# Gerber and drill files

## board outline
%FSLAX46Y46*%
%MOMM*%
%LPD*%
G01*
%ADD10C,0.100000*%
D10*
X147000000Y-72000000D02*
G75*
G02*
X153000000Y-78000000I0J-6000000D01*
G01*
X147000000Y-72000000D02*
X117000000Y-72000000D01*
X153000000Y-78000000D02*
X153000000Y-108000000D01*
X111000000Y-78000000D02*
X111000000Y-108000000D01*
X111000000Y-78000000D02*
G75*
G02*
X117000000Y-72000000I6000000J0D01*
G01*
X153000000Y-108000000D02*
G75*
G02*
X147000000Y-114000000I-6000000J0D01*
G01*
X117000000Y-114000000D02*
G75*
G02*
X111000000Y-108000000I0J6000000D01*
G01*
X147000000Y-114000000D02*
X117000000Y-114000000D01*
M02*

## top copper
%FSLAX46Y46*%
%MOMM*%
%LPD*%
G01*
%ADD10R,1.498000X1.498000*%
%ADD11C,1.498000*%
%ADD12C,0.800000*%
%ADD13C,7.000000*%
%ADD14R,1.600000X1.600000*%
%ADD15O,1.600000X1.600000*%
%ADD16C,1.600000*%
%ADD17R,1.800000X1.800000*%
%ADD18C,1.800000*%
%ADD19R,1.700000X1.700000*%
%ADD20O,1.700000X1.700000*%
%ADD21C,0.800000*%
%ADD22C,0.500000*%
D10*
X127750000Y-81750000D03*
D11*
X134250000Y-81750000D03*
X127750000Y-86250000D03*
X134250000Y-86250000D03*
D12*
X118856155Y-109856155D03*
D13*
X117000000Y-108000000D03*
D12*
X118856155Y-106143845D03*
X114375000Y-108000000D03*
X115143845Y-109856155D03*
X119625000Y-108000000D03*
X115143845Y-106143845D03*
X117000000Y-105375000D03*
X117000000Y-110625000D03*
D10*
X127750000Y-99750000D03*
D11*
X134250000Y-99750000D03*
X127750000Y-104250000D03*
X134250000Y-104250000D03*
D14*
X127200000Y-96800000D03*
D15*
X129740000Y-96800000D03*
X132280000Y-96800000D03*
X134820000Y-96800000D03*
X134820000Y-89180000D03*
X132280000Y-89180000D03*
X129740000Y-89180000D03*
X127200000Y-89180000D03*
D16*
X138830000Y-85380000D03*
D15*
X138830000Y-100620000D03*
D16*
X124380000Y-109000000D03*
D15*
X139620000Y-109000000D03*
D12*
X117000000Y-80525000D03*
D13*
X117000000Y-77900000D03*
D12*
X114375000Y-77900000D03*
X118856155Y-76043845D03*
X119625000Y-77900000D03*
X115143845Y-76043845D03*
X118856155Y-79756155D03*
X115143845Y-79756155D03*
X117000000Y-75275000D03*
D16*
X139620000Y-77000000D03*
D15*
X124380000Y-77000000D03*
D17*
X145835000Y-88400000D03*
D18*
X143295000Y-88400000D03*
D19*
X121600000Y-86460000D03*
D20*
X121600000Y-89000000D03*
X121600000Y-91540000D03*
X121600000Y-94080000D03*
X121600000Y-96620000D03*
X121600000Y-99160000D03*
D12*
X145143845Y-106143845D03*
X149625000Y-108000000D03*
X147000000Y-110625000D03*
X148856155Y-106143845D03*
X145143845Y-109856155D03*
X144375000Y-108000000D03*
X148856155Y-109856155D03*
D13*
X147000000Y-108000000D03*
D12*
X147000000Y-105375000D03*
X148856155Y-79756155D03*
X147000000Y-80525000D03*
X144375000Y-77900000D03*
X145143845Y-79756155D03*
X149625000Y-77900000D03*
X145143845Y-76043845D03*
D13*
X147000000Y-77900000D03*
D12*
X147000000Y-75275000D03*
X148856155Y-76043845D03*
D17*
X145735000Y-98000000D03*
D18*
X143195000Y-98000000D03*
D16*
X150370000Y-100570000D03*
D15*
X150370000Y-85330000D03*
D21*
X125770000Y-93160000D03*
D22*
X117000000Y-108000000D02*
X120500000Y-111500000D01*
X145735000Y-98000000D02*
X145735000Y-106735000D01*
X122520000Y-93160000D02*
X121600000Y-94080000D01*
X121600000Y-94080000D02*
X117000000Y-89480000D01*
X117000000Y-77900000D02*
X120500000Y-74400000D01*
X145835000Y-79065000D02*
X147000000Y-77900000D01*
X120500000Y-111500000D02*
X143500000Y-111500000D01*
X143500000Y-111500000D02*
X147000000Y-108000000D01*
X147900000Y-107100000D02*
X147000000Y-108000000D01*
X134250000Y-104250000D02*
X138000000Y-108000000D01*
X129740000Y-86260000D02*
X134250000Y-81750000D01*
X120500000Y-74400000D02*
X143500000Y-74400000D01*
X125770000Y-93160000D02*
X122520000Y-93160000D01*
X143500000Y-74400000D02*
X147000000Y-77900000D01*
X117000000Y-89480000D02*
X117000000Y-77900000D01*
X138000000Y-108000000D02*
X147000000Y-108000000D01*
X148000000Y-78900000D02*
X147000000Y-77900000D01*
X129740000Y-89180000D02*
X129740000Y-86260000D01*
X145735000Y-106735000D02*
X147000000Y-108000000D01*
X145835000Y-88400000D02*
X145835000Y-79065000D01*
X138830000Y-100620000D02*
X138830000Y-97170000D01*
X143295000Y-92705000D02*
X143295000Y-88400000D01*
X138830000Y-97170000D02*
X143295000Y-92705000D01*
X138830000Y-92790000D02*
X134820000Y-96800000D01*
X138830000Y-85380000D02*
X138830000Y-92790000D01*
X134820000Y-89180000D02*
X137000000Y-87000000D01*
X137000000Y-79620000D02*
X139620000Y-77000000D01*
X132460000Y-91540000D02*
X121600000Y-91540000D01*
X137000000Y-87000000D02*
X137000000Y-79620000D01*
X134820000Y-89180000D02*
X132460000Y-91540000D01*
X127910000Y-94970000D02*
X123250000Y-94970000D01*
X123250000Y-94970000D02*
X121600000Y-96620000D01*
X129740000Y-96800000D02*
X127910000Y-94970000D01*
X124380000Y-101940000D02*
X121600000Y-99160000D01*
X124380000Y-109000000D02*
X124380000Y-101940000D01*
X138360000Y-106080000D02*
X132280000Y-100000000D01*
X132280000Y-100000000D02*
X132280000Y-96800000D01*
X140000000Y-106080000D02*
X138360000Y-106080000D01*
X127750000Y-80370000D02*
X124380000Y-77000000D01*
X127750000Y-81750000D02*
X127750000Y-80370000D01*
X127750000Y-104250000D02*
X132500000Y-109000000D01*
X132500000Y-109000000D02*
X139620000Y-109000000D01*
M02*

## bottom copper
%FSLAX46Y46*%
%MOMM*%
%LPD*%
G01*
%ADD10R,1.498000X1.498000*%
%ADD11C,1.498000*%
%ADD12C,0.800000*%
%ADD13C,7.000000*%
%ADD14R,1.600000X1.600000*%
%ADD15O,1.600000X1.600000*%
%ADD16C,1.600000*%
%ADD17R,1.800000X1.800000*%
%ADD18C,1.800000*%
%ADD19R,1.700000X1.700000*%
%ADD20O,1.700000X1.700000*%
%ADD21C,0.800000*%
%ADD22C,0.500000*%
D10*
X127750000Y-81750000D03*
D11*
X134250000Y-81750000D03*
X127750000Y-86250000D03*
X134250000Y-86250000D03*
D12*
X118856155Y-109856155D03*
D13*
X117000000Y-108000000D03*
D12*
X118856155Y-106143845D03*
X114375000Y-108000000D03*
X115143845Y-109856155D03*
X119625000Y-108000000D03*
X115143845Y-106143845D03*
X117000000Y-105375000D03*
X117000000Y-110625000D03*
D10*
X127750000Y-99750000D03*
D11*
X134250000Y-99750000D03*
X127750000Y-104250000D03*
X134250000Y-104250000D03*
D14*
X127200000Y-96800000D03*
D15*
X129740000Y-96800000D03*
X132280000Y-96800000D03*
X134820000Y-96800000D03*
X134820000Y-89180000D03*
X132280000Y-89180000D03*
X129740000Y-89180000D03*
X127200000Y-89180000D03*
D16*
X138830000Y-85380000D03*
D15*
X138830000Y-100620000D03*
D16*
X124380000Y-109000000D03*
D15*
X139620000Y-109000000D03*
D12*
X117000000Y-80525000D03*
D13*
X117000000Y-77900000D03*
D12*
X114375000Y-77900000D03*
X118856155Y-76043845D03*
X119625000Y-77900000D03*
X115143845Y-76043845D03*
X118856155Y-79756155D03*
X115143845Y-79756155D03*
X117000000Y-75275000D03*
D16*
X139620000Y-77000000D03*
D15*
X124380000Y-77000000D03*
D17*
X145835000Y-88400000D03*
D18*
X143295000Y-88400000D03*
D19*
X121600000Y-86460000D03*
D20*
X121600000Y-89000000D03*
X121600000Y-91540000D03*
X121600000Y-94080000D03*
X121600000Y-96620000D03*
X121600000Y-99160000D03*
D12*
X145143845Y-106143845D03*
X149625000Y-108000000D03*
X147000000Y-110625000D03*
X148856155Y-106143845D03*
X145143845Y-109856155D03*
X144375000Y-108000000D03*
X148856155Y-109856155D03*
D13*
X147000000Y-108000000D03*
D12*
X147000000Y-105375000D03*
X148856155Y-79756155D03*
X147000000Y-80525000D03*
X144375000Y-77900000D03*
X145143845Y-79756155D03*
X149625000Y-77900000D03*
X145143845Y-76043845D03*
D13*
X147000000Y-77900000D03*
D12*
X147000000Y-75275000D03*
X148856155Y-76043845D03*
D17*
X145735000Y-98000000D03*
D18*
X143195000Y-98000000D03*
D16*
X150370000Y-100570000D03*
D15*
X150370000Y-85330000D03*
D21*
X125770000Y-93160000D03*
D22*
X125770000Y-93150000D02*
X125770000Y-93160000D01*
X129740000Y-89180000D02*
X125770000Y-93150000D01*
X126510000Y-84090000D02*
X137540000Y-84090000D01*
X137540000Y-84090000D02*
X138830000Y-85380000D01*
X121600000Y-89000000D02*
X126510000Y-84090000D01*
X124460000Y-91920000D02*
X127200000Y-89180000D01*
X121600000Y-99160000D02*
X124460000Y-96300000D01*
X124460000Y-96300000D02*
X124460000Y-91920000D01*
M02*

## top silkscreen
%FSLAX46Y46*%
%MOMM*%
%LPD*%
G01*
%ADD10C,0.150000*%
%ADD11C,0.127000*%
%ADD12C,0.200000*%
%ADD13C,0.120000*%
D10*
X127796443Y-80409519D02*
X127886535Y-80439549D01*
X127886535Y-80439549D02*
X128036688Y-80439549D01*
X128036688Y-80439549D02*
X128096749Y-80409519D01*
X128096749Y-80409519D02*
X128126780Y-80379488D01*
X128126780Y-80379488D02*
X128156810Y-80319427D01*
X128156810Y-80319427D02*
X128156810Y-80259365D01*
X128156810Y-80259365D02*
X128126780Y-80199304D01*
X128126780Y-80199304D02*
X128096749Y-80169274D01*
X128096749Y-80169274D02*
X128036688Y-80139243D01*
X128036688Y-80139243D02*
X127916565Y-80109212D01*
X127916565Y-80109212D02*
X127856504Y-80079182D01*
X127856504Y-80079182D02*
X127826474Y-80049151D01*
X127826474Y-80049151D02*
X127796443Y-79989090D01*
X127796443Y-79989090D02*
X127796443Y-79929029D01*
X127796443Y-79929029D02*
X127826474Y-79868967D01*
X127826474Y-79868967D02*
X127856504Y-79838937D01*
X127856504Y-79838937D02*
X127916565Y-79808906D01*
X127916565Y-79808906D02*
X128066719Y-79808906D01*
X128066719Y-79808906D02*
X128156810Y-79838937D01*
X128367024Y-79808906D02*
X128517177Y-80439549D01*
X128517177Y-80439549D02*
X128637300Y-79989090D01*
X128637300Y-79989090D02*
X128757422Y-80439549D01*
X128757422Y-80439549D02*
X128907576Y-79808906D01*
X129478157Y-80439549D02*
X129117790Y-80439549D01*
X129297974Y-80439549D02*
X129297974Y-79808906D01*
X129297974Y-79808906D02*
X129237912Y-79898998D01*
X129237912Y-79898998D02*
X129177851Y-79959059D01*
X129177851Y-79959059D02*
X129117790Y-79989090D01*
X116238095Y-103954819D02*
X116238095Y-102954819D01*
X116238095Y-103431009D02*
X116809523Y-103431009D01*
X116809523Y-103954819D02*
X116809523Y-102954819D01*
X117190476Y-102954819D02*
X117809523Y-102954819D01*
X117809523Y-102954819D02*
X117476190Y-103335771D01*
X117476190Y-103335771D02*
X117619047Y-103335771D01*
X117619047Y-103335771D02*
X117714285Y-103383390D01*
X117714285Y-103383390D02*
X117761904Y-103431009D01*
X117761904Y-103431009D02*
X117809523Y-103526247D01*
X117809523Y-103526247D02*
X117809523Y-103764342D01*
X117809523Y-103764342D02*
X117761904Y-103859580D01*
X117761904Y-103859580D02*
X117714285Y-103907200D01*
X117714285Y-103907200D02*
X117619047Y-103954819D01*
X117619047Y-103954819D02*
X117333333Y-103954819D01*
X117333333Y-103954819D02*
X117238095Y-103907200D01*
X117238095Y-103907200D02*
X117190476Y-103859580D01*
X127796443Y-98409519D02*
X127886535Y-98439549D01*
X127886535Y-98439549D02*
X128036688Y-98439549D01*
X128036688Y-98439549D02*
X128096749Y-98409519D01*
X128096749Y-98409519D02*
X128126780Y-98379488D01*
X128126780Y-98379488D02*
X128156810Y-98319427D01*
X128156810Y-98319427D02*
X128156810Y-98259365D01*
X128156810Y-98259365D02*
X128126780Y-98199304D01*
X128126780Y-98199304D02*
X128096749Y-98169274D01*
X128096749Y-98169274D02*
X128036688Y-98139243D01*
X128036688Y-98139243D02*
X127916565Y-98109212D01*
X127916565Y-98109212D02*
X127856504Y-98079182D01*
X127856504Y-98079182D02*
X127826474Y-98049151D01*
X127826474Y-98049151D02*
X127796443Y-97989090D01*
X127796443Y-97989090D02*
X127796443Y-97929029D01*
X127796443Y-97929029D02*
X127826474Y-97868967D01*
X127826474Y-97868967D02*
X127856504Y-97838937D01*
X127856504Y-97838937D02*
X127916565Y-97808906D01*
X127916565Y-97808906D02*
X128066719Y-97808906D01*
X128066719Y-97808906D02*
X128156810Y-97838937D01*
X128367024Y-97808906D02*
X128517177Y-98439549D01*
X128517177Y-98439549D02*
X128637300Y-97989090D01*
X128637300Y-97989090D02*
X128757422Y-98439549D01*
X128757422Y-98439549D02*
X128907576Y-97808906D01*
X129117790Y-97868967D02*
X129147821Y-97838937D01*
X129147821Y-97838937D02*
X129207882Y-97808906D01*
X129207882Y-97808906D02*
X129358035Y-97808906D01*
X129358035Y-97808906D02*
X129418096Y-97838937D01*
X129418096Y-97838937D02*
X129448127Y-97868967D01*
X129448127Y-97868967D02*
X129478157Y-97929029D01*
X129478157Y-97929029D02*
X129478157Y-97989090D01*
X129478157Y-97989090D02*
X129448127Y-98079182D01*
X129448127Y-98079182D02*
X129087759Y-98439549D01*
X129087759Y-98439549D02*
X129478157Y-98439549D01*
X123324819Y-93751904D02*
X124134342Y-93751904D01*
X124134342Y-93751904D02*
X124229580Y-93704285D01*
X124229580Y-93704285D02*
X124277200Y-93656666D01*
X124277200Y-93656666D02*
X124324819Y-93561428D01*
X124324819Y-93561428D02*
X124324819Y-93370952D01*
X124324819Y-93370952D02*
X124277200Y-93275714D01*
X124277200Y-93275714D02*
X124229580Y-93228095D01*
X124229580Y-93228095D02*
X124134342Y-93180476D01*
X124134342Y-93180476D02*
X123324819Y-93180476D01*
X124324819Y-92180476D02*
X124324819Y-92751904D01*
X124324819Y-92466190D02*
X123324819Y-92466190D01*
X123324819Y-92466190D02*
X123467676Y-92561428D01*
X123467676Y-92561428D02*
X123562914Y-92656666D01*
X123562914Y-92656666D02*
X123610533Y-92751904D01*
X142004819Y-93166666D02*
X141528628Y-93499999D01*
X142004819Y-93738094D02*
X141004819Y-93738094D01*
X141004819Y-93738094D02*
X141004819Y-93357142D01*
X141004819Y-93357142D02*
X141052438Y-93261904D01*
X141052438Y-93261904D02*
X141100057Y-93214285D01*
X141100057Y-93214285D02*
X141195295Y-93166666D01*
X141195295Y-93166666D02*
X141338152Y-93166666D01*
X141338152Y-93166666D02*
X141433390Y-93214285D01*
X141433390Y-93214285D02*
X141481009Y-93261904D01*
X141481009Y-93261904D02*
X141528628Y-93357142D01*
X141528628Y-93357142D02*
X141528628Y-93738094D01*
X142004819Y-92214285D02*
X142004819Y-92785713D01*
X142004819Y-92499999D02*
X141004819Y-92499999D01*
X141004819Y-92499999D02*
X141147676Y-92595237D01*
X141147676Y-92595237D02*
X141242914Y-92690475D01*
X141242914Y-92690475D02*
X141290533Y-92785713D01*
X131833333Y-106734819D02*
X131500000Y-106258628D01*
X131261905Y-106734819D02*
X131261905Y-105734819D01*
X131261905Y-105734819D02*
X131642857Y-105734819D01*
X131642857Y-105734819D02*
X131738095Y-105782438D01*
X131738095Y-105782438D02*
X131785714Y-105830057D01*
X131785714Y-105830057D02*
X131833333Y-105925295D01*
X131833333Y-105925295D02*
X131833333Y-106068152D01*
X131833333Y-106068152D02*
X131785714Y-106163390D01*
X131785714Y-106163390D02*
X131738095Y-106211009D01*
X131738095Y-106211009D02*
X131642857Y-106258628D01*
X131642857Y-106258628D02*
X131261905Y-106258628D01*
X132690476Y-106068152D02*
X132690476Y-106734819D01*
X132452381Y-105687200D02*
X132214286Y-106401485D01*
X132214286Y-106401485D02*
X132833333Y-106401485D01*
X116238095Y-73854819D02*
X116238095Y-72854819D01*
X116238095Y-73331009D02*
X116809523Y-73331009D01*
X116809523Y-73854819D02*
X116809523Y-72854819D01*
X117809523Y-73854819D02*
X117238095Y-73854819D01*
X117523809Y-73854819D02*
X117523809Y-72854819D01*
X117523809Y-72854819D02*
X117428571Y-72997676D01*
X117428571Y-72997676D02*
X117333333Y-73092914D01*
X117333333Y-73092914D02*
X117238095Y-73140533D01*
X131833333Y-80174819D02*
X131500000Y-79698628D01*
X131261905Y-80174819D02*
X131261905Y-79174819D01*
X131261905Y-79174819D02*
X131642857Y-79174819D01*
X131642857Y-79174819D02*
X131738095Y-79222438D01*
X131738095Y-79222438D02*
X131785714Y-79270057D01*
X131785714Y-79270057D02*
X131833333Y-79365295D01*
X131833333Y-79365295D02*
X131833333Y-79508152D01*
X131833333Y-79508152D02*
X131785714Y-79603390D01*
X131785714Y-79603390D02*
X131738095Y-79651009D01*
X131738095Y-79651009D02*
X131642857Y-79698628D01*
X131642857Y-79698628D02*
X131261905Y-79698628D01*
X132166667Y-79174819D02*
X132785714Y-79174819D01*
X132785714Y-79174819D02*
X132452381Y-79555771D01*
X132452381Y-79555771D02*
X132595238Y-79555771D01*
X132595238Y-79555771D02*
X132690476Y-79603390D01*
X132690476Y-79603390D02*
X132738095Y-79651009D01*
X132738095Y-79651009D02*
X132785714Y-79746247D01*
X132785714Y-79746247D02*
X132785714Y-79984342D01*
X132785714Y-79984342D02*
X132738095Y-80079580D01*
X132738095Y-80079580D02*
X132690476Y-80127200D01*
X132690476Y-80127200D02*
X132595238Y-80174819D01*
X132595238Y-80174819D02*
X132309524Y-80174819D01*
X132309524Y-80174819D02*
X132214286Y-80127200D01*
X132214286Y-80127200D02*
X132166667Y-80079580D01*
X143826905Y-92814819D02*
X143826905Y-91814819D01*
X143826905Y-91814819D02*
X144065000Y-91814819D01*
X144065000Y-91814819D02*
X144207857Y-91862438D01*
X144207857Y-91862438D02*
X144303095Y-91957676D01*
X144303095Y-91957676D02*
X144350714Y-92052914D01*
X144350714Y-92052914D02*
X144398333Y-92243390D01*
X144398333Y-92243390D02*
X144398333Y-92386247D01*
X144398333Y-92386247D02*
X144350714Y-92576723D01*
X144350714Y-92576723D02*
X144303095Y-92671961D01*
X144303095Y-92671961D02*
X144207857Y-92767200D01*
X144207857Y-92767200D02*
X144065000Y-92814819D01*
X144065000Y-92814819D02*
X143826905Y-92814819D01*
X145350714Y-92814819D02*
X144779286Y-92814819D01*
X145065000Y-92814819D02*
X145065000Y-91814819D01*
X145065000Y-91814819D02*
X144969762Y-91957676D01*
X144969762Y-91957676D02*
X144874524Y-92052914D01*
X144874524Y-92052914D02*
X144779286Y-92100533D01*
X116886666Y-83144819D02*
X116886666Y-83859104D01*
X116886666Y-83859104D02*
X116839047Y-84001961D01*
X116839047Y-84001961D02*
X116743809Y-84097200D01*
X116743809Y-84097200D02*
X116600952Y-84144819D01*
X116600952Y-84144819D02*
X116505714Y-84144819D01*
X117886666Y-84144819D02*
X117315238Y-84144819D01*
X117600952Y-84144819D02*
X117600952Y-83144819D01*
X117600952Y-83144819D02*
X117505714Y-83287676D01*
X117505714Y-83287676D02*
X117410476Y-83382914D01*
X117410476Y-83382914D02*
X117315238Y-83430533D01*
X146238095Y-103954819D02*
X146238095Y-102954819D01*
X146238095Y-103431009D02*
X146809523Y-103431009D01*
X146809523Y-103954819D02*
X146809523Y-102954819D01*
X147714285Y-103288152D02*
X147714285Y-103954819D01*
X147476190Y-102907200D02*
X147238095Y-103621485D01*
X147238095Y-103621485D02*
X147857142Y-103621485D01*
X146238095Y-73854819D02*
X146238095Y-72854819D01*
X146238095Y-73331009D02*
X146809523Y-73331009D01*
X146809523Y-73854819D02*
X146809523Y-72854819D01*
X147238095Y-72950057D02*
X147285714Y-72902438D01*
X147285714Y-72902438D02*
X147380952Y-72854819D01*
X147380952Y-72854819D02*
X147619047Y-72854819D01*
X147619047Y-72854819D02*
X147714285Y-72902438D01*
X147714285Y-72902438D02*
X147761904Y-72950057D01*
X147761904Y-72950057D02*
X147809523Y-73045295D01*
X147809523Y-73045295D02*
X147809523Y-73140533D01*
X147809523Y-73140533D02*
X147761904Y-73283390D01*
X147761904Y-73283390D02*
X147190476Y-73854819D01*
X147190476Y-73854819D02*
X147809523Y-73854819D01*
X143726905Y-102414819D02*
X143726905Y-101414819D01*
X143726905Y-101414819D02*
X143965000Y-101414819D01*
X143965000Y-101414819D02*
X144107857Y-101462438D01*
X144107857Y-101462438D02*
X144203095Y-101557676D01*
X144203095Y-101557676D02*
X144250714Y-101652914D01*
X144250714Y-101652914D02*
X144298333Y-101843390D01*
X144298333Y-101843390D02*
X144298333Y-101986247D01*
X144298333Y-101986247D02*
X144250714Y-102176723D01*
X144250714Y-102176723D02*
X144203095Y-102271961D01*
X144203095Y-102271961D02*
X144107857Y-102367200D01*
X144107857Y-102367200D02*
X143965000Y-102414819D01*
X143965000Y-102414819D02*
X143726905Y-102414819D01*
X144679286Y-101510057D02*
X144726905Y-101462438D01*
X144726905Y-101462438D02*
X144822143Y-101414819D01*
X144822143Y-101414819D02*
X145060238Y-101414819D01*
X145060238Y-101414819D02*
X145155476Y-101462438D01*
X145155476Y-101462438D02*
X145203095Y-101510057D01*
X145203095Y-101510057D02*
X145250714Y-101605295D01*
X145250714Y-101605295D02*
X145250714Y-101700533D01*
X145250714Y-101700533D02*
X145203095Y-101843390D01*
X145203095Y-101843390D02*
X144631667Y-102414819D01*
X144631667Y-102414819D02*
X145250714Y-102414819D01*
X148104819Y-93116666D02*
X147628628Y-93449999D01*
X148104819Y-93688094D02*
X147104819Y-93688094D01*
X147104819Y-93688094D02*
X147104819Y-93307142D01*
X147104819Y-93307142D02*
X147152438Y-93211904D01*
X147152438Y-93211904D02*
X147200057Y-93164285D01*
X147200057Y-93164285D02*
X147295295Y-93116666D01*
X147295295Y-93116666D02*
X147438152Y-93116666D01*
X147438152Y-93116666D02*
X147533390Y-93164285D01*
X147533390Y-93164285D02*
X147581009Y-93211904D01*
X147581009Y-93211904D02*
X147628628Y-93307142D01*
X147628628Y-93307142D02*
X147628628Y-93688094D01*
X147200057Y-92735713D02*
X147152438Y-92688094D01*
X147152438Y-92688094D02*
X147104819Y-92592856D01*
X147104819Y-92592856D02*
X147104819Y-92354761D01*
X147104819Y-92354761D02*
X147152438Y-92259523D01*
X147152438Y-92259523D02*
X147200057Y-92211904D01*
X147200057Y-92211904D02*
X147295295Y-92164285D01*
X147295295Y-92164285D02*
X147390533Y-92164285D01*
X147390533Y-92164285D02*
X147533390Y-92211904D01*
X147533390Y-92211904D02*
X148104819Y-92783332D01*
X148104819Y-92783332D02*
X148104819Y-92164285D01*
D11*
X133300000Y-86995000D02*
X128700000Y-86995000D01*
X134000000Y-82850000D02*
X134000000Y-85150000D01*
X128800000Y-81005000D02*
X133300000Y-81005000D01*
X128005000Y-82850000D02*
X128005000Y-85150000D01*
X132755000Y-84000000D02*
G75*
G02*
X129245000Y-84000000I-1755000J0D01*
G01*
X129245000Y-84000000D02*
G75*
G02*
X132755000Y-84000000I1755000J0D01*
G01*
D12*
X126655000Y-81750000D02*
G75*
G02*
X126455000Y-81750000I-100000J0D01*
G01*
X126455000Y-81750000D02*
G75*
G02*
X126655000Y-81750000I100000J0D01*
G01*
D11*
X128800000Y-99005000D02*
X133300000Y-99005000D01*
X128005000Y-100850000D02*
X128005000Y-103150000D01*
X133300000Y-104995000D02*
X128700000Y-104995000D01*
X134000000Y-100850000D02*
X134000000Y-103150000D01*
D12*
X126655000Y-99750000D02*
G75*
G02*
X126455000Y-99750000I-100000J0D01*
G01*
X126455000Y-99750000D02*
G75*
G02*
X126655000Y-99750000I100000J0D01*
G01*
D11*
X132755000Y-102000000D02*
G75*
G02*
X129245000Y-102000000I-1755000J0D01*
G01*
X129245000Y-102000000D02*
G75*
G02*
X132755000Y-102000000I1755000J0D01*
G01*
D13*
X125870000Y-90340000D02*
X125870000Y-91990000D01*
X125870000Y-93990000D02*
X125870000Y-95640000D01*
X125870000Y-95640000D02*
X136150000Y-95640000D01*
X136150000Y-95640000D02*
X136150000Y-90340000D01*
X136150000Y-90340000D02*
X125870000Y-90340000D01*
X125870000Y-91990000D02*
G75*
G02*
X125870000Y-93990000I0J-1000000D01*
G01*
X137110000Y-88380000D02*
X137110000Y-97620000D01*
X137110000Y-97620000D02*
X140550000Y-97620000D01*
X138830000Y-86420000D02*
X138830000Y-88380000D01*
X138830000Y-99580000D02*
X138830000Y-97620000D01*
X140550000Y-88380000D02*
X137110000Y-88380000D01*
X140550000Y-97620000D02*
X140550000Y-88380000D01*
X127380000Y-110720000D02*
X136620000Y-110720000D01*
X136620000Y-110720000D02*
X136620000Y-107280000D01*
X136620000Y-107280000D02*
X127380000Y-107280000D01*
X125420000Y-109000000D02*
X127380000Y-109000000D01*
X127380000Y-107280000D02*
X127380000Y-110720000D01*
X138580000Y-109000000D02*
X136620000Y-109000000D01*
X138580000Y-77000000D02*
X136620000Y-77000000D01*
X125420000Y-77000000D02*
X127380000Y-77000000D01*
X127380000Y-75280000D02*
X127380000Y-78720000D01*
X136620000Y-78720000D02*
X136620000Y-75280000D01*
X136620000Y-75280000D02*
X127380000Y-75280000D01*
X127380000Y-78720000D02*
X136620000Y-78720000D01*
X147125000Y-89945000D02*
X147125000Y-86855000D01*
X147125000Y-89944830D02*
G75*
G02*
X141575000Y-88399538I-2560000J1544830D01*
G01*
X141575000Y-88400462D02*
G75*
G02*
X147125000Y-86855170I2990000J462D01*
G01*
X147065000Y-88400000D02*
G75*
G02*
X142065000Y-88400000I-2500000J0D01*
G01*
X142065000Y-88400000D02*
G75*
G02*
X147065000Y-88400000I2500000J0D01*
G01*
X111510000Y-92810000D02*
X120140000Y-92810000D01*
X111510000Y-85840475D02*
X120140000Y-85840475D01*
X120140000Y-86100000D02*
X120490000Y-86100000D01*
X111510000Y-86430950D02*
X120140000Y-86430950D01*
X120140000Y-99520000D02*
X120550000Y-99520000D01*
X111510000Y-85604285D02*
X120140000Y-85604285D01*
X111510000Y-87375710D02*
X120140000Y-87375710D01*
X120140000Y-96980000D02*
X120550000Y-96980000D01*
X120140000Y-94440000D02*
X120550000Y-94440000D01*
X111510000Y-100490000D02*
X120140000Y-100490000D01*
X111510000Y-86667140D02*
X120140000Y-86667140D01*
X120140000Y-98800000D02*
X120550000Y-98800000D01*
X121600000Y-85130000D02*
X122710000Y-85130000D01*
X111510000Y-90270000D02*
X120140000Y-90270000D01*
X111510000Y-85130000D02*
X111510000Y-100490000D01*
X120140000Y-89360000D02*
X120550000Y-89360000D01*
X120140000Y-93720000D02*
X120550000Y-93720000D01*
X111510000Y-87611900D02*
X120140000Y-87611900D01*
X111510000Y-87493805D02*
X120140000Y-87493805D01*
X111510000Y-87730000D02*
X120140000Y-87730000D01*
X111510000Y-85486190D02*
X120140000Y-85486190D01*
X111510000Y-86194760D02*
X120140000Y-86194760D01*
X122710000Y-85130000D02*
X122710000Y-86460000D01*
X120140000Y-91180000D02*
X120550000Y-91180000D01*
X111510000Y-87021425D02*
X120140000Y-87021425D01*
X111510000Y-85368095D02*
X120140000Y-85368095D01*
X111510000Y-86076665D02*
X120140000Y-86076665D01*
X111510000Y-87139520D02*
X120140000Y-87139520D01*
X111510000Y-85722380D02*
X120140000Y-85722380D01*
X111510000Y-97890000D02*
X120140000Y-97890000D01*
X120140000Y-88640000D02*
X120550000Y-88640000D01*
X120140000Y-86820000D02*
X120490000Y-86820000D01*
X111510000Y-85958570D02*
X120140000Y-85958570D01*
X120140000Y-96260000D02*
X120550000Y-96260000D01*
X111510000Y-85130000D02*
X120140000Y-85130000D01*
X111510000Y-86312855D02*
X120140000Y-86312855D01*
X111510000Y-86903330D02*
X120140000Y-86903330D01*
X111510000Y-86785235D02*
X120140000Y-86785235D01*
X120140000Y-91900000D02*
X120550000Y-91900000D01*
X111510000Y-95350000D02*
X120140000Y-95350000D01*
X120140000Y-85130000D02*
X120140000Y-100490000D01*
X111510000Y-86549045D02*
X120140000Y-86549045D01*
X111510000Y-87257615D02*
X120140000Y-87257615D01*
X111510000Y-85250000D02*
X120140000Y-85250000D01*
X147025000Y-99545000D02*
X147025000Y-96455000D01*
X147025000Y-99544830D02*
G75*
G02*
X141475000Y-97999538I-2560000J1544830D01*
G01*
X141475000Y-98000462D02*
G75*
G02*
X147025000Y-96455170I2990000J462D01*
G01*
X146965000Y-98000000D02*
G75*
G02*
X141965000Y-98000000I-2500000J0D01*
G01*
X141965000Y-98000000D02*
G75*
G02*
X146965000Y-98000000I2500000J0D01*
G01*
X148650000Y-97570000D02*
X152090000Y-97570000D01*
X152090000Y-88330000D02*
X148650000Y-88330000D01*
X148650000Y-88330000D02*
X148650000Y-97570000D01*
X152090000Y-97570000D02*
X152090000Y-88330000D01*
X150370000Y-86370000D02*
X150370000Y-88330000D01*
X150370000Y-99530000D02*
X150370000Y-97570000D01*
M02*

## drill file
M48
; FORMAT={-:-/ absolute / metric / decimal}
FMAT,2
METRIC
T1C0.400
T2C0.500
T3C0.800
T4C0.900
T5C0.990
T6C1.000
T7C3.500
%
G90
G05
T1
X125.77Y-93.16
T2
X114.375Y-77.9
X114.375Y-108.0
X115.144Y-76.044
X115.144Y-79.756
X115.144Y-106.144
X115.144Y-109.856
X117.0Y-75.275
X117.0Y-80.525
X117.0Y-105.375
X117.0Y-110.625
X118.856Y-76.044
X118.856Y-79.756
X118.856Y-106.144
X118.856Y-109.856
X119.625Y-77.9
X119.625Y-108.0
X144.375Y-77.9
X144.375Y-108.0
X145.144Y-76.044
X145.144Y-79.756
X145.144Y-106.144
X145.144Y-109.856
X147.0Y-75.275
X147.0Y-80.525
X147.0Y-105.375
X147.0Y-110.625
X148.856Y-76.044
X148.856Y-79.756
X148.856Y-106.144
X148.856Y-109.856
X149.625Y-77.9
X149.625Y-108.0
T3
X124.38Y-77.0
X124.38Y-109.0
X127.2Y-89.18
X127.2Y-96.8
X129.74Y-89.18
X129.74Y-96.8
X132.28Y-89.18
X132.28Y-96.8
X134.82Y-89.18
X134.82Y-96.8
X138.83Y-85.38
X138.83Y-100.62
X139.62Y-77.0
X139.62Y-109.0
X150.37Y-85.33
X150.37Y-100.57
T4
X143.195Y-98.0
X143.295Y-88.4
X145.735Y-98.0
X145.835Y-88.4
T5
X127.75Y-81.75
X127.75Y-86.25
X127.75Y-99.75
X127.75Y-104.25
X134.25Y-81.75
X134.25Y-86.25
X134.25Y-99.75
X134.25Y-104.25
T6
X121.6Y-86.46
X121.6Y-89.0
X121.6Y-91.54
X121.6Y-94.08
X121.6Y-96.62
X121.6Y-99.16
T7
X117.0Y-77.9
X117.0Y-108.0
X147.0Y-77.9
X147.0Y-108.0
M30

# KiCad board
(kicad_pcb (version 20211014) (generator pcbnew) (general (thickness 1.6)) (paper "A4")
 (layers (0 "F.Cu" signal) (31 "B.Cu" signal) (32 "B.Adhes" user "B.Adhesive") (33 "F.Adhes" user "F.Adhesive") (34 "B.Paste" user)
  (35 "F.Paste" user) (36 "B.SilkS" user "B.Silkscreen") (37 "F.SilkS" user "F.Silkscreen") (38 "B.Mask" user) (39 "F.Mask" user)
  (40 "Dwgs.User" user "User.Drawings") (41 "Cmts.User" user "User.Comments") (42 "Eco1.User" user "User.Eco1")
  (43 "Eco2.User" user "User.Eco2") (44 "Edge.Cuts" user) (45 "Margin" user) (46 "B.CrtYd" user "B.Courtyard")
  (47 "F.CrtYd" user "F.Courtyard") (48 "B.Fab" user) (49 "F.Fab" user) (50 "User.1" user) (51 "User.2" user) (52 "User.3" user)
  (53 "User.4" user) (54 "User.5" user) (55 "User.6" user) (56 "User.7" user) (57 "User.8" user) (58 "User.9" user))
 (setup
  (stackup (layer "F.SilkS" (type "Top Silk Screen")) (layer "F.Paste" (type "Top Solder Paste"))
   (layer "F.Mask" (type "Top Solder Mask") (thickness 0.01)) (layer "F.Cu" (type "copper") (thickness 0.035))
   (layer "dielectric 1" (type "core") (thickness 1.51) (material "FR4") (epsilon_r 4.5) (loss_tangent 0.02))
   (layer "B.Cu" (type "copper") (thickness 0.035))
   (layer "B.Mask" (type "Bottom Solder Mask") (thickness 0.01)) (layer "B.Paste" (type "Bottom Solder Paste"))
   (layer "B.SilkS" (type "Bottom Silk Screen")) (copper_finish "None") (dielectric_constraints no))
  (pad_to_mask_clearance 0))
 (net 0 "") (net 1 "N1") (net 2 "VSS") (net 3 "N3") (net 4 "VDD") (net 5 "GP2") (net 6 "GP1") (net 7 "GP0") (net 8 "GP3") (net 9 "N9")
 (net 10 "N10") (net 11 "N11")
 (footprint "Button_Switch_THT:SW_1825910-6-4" (layer "F.Cu") (at 131 84)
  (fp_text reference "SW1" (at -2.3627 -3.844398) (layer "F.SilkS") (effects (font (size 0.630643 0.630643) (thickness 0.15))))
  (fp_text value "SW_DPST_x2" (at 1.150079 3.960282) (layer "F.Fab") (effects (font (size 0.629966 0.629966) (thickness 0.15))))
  (fp_line (start 2.3 2.995) (end -2.3 2.995) (layer "F.SilkS") (width 0.127))
  (fp_line (start 3 -1.15) (end 3 1.15) (layer "F.SilkS") (width 0.127))
  (fp_line (start -2.2 -2.995) (end 2.3 -2.995) (layer "F.SilkS") (width 0.127))
  (fp_line (start -2.995 -1.15) (end -2.995 1.15) (layer "F.SilkS") (width 0.127))
  (fp_circle (center 0 0) (end 1.755 0) (layer "F.SilkS") (width 0.127) (fill none))
  (fp_circle (center -4.445 -2.25) (end -4.345 -2.25) (layer "F.SilkS") (width 0.2) (fill none))
  (pad "1" thru_hole rect locked (at -3.25 -2.25) (size 1.498 1.498) (drill 0.99) (layers *.Cu *.Mask) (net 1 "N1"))
  (pad "2" thru_hole circle locked (at 3.25 -2.25) (size 1.498 1.498) (drill 0.99) (layers *.Cu *.Mask) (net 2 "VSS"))
  (pad "3" thru_hole circle locked (at -3.25 2.25) (size 1.498 1.498) (drill 0.99) (layers *.Cu *.Mask))
  (pad "4" thru_hole circle locked (at 3.25 2.25) (size 1.498 1.498) (drill 0.99) (layers *.Cu *.Mask)))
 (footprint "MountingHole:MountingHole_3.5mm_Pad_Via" (layer "F.Cu") (at 117 108)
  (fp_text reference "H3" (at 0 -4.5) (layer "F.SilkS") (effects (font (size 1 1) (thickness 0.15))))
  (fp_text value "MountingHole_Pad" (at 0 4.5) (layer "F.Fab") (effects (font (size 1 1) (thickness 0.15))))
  (pad "1" thru_hole circle (at 1.856155 1.856155) (size 0.8 0.8) (drill 0.5) (layers *.Cu *.Mask) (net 2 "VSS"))
  (pad "1" thru_hole circle (at 0 0) (size 7 7) (drill 3.5) (layers *.Cu *.Mask) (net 2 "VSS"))
  (pad "1" thru_hole circle (at 1.856155 -1.856155) (size 0.8 0.8) (drill 0.5) (layers *.Cu *.Mask) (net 2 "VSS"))
  (pad "1" thru_hole circle (at -2.625 0) (size 0.8 0.8) (drill 0.5) (layers *.Cu *.Mask) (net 2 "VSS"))
  (pad "1" thru_hole circle (at -1.856155 1.856155) (size 0.8 0.8) (drill 0.5) (layers *.Cu *.Mask) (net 2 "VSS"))
  (pad "1" thru_hole circle (at 2.625 0) (size 0.8 0.8) (drill 0.5) (layers *.Cu *.Mask) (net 2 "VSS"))
  (pad "1" thru_hole circle (at -1.856155 -1.856155) (size 0.8 0.8) (drill 0.5) (layers *.Cu *.Mask) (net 2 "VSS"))
  (pad "1" thru_hole circle (at 0 -2.625) (size 0.8 0.8) (drill 0.5) (layers *.Cu *.Mask) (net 2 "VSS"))
  (pad "1" thru_hole circle (at 0 2.625) (size 0.8 0.8) (drill 0.5) (layers *.Cu *.Mask) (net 2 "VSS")))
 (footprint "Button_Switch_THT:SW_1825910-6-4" (layer "F.Cu") (at 131 102)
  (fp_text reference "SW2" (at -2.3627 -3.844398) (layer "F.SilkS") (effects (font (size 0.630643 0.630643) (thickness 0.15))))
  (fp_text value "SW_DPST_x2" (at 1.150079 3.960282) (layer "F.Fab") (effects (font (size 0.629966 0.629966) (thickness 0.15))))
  (fp_line (start -2.2 -2.995) (end 2.3 -2.995) (layer "F.SilkS") (width 0.127))
  (fp_line (start -2.995 -1.15) (end -2.995 1.15) (layer "F.SilkS") (width 0.127))
  (fp_line (start 2.3 2.995) (end -2.3 2.995) (layer "F.SilkS") (width 0.127))
  (fp_line (start 3 -1.15) (end 3 1.15) (layer "F.SilkS") (width 0.127))
  (fp_circle (center -4.445 -2.25) (end -4.345 -2.25) (layer "F.SilkS") (width 0.2) (fill none))
  (fp_circle (center 0 0) (end 1.755 0) (layer "F.SilkS") (width 0.127) (fill none))
  (pad "1" thru_hole rect locked (at -3.25 -2.25) (size 1.498 1.498) (drill 0.99) (layers *.Cu *.Mask))
  (pad "2" thru_hole circle locked (at 3.25 -2.25) (size 1.498 1.498) (drill 0.99) (layers *.Cu *.Mask))
  (pad "3" thru_hole circle locked (at -3.25 2.25) (size 1.498 1.498) (drill 0.99) (layers *.Cu *.Mask) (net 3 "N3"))
  (pad "4" thru_hole circle locked (at 3.25 2.25) (size 1.498 1.498) (drill 0.99) (layers *.Cu *.Mask) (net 2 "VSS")))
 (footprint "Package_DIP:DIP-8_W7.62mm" (layer "F.Cu") (at 127.2 96.8 90)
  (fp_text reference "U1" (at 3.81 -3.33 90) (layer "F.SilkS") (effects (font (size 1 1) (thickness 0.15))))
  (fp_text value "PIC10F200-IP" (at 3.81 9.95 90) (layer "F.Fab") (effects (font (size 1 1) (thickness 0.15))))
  (fp_line (start 6.46 -1.33) (end 4.81 -1.33) (layer "F.SilkS") (width 0.12))
  (fp_line (start 2.81 -1.33) (end 1.16 -1.33) (layer "F.SilkS") (width 0.12))
  (fp_line (start 1.16 -1.33) (end 1.16 8.95) (layer "F.SilkS") (width 0.12))
  (fp_line (start 1.16 8.95) (end 6.46 8.95) (layer "F.SilkS") (width 0.12))
  (fp_line (start 6.46 8.95) (end 6.46 -1.33) (layer "F.SilkS") (width 0.12))
  (fp_arc (start 4.81 -1.33) (mid 3.81 -0.33) (end 2.81 -1.33) (layer "F.SilkS") (width 0.12))
  (pad "1" thru_hole rect (at 0 0 90) (size 1.6 1.6) (drill 0.8) (layers *.Cu *.Mask))
  (pad "2" thru_hole oval (at 0 2.54 90) (size 1.6 1.6) (drill 0.8) (layers *.Cu *.Mask) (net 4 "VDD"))
  (pad "3" thru_hole oval (at 0 5.08 90) (size 1.6 1.6) (drill 0.8) (layers *.Cu *.Mask) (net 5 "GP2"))
  (pad "4" thru_hole oval (at 0 7.62 90) (size 1.6 1.6) (drill 0.8) (layers *.Cu *.Mask) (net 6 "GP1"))
  (pad "5" thru_hole oval (at 7.62 7.62 90) (size 1.6 1.6) (drill 0.8) (layers *.Cu *.Mask) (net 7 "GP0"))
  (pad "6" thru_hole oval (at 7.62 5.08 90) (size 1.6 1.6) (drill 0.8) (layers *.Cu *.Mask))
  (pad "7" thru_hole oval (at 7.62 2.54 90) (size 1.6 1.6) (drill 0.8) (layers *.Cu *.Mask) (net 2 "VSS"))
  (pad "8" thru_hole oval (at 7.62 0 90) (size 1.6 1.6) (drill 0.8) (layers *.Cu *.Mask) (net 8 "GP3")))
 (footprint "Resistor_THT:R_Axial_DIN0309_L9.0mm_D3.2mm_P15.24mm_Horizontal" (layer "F.Cu") (at 138.83 85.38 -90)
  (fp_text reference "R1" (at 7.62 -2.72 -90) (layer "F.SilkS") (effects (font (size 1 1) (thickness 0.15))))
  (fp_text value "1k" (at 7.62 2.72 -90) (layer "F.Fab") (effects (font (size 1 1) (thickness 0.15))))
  (fp_line (start 3 1.72) (end 12.24 1.72) (layer "F.SilkS") (width 0.12))
  (fp_line (start 12.24 1.72) (end 12.24 -1.72) (layer "F.SilkS") (width 0.12))
  (fp_line (start 1.04 0) (end 3 0) (layer "F.SilkS") (width 0.12))
  (fp_line (start 14.2 0) (end 12.24 0) (layer "F.SilkS") (width 0.12))
  (fp_line (start 3 -1.72) (end 3 1.72) (layer "F.SilkS") (width 0.12))
  (fp_line (start 12.24 -1.72) (end 3 -1.72) (layer "F.SilkS") (width 0.12))
  (pad "1" thru_hole circle (at 0 0 270) (size 1.6 1.6) (drill 0.8) (layers *.Cu *.Mask) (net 6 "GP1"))
  (pad "2" thru_hole oval (at 15.24 0 270) (size 1.6 1.6) (drill 0.8) (layers *.Cu *.Mask) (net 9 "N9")))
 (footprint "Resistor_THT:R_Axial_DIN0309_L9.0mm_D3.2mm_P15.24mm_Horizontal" (layer "F.Cu") (at 124.38 109)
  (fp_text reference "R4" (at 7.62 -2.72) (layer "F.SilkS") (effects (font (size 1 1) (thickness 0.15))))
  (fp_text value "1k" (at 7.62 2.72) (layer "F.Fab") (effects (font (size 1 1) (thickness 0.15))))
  (fp_line (start 3 1.72) (end 12.24 1.72) (layer "F.SilkS") (width 0.12))
  (fp_line (start 12.24 1.72) (end 12.24 -1.72) (layer "F.SilkS") (width 0.12))
  (fp_line (start 12.24 -1.72) (end 3 -1.72) (layer "F.SilkS") (width 0.12))
  (fp_line (start 1.04 0) (end 3 0) (layer "F.SilkS") (width 0.12))
  (fp_line (start 3 -1.72) (end 3 1.72) (layer "F.SilkS") (width 0.12))
  (fp_line (start 14.2 0) (end 12.24 0) (layer "F.SilkS") (width 0.12))
  (pad "1" thru_hole circle (at 0 0) (size 1.6 1.6) (drill 0.8) (layers *.Cu *.Mask) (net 8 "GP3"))
  (pad "2" thru_hole oval (at 15.24 0) (size 1.6 1.6) (drill 0.8) (layers *.Cu *.Mask) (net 3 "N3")))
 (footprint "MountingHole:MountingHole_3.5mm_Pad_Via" (layer "F.Cu") (at 117 77.9)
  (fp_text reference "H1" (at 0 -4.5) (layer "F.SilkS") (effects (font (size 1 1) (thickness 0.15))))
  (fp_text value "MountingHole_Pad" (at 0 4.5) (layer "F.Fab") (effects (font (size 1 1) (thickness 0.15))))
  (pad "1" thru_hole circle (at 0 2.625) (size 0.8 0.8) (drill 0.5) (layers *.Cu *.Mask) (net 2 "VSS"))
  (pad "1" thru_hole circle (at 0 0) (size 7 7) (drill 3.5) (layers *.Cu *.Mask) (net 2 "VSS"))
  (pad "1" thru_hole circle (at -2.625 0) (size 0.8 0.8) (drill 0.5) (layers *.Cu *.Mask) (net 2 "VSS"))
  (pad "1" thru_hole circle (at 1.856155 -1.856155) (size 0.8 0.8) (drill 0.5) (layers *.Cu *.Mask) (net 2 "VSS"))
  (pad "1" thru_hole circle (at 2.625 0) (size 0.8 0.8) (drill 0.5) (layers *.Cu *.Mask) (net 2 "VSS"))
  (pad "1" thru_hole circle (at -1.856155 -1.856155) (size 0.8 0.8) (drill 0.5) (layers *.Cu *.Mask) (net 2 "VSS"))
  (pad "1" thru_hole circle (at 1.856155 1.856155) (size 0.8 0.8) (drill 0.5) (layers *.Cu *.Mask) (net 2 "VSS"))
  (pad "1" thru_hole circle (at -1.856155 1.856155) (size 0.8 0.8) (drill 0.5) (layers *.Cu *.Mask) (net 2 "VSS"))
  (pad "1" thru_hole circle (at 0 -2.625) (size 0.8 0.8) (drill 0.5) (layers *.Cu *.Mask) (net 2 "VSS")))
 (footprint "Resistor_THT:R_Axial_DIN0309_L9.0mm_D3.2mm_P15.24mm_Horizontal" (layer "F.Cu") (at 139.62 77 180)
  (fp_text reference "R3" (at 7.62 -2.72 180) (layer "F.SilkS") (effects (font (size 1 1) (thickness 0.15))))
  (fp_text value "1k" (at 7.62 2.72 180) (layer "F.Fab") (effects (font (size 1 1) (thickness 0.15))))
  (fp_line (start 1.04 0) (end 3 0) (layer "F.SilkS") (width 0.12))
  (fp_line (start 14.2 0) (end 12.24 0) (layer "F.SilkS") (width 0.12))
  (fp_line (start 12.24 1.72) (end 12.24 -1.72) (layer "F.SilkS") (width 0.12))
  (fp_line (start 3 -1.72) (end 3 1.72) (layer "F.SilkS") (width 0.12))
  (fp_line (start 3 1.72) (end 12.24 1.72) (layer "F.SilkS") (width 0.12))
  (fp_line (start 12.24 -1.72) (end 3 -1.72) (layer "F.SilkS") (width 0.12))
  (pad "1" thru_hole circle (at 0 0 180) (size 1.6 1.6) (drill 0.8) (layers *.Cu *.Mask) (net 7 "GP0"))
  (pad "2" thru_hole oval (at 15.24 0 180) (size 1.6 1.6) (drill 0.8) (layers *.Cu *.Mask) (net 1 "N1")))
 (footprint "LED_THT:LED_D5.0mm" (layer "F.Cu") (at 145.835 88.4 180)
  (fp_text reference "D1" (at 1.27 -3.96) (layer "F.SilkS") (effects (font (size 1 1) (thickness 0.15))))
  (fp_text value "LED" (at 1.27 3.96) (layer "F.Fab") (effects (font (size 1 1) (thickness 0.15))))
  (fp_line (start -1.29 -1.545) (end -1.29 1.545) (layer "F.SilkS") (width 0.12))
  (fp_arc (start -1.29 -1.54483) (mid 2.072002 -2.880433) (end 4.26 0.000462) (layer "F.SilkS") (width 0.12))
  (fp_arc (start 4.26 -0.000462) (mid 2.072002 2.880433) (end -1.29 1.54483) (layer "F.SilkS") (width 0.12))
  (fp_circle (center 1.27 0) (end 3.77 0) (layer "F.SilkS") (width 0.12) (fill none))
  (pad "1" thru_hole rect (at 0 0 180) (size 1.8 1.8) (drill 0.9) (layers *.Cu *.Mask) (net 2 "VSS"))
  (pad "2" thru_hole circle (at 2.54 0 180) (size 1.8 1.8) (drill 0.9) (layers *.Cu *.Mask) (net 9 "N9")))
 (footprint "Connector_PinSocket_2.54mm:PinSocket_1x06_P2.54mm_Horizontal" (layer "F.Cu") (at 121.6 86.46)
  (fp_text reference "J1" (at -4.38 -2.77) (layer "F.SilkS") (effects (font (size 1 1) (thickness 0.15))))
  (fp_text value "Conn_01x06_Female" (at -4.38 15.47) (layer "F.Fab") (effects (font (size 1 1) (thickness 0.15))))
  (fp_line (start -10.09 6.35) (end -1.46 6.35) (layer "F.SilkS") (width 0.12))
  (fp_line (start -10.09 -0.619525) (end -1.46 -0.619525) (layer "F.SilkS") (width 0.12))
  (fp_line (start -1.46 -0.36) (end -1.11 -0.36) (layer "F.SilkS") (width 0.12))
  (fp_line (start -10.09 -0.02905) (end -1.46 -0.02905) (layer "F.SilkS") (width 0.12))
  (fp_line (start -1.46 13.06) (end -1.05 13.06) (layer "F.SilkS") (width 0.12))
  (fp_line (start -10.09 -0.855715) (end -1.46 -0.855715) (layer "F.SilkS") (width 0.12))
  (fp_line (start -10.09 0.91571) (end -1.46 0.91571) (layer "F.SilkS") (width 0.12))
  (fp_line (start -1.46 10.52) (end -1.05 10.52) (layer "F.SilkS") (width 0.12))
  (fp_line (start -1.46 7.98) (end -1.05 7.98) (layer "F.SilkS") (width 0.12))
  (fp_line (start -10.09 14.03) (end -1.46 14.03) (layer "F.SilkS") (width 0.12))
  (fp_line (start -10.09 0.20714) (end -1.46 0.20714) (layer "F.SilkS") (width 0.12))
  (fp_line (start -1.46 12.34) (end -1.05 12.34) (layer "F.SilkS") (width 0.12))
  (fp_line (start 0 -1.33) (end 1.11 -1.33) (layer "F.SilkS") (width 0.12))
  (fp_line (start -10.09 3.81) (end -1.46 3.81) (layer "F.SilkS") (width 0.12))
  (fp_line (start -10.09 -1.33) (end -10.09 14.03) (layer "F.SilkS") (width 0.12))
  (fp_line (start -1.46 2.9) (end -1.05 2.9) (layer "F.SilkS") (width 0.12))
  (fp_line (start -1.46 7.26) (end -1.05 7.26) (layer "F.SilkS") (width 0.12))
  (fp_line (start -10.09 1.1519) (end -1.46 1.1519) (layer "F.SilkS") (width 0.12))
  (fp_line (start -10.09 1.033805) (end -1.46 1.033805) (layer "F.SilkS") (width 0.12))
  (fp_line (start -10.09 1.27) (end -1.46 1.27) (layer "F.SilkS") (width 0.12))
  (fp_line (start -10.09 -0.97381) (end -1.46 -0.97381) (layer "F.SilkS") (width 0.12))
  (fp_line (start -10.09 -0.26524) (end -1.46 -0.26524) (layer "F.SilkS") (width 0.12))
  (fp_line (start 1.11 -1.33) (end 1.11 0) (layer "F.SilkS") (width 0.12))
  (fp_line (start -1.46 4.72) (end -1.05 4.72) (layer "F.SilkS") (width 0.12))
  (fp_line (start -10.09 0.561425) (end -1.46 0.561425) (layer "F.SilkS") (width 0.12))
  (fp_line (start -10.09 -1.091905) (end -1.46 -1.091905) (layer "F.SilkS") (width 0.12))
  (fp_line (start -10.09 -0.383335) (end -1.46 -0.383335) (layer "F.SilkS") (width 0.12))
  (fp_line (start -10.09 0.67952) (end -1.46 0.67952) (layer "F.SilkS") (width 0.12))
  (fp_line (start -10.09 -0.73762) (end -1.46 -0.73762) (layer "F.SilkS") (width 0.12))
  (fp_line (start -10.09 11.43) (end -1.46 11.43) (layer "F.SilkS") (width 0.12))
  (fp_line (start -1.46 2.18) (end -1.05 2.18) (layer "F.SilkS") (width 0.12))
  (fp_line (start -1.46 0.36) (end -1.11 0.36) (layer "F.SilkS") (width 0.12))
  (fp_line (start -10.09 -0.50143) (end -1.46 -0.50143) (layer "F.SilkS") (width 0.12))
  (fp_line (start -1.46 9.8) (end -1.05 9.8) (layer "F.SilkS") (width 0.12))
  (fp_line (start -10.09 -1.33) (end -1.46 -1.33) (layer "F.SilkS") (width 0.12))
  (fp_line (start -10.09 -0.147145) (end -1.46 -0.147145) (layer "F.SilkS") (width 0.12))
  (fp_line (start -10.09 0.44333) (end -1.46 0.44333) (layer "F.SilkS") (width 0.12))
  (fp_line (start -10.09 0.325235) (end -1.46 0.325235) (layer "F.SilkS") (width 0.12))
  (fp_line (start -1.46 5.44) (end -1.05 5.44) (layer "F.SilkS") (width 0.12))
  (fp_line (start -10.09 8.89) (end -1.46 8.89) (layer "F.SilkS") (width 0.12))
  (fp_line (start -1.46 -1.33) (end -1.46 14.03) (layer "F.SilkS") (width 0.12))
  (fp_line (start -10.09 0.089045) (end -1.46 0.089045) (layer "F.SilkS") (width 0.12))
  (fp_line (start -10.09 0.797615) (end -1.46 0.797615) (layer "F.SilkS") (width 0.12))
  (fp_line (start -10.09 -1.21) (end -1.46 -1.21) (layer "F.SilkS") (width 0.12))
  (pad "1" thru_hole rect (at 0 0) (size 1.7 1.7) (drill 1) (layers *.Cu *.Mask) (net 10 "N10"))
  (pad "2" thru_hole oval (at 0 2.54) (size 1.7 1.7) (drill 1) (layers *.Cu *.Mask) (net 6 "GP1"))
  (pad "3" thru_hole oval (at 0 5.08) (size 1.7 1.7) (drill 1) (layers *.Cu *.Mask) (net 7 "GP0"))
  (pad "4" thru_hole oval (at 0 7.62) (size 1.7 1.7) (drill 1) (layers *.Cu *.Mask) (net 2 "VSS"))
  (pad "5" thru_hole oval (at 0 10.16) (size 1.7 1.7) (drill 1) (layers *.Cu *.Mask) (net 4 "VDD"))
  (pad "6" thru_hole oval (at 0 12.7) (size 1.7 1.7) (drill 1) (layers *.Cu *.Mask) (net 8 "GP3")))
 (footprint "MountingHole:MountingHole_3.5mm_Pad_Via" (layer "F.Cu") (at 147 108)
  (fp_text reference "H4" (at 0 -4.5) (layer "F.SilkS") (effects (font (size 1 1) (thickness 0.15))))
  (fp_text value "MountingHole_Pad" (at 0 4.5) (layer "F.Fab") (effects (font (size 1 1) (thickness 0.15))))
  (pad "1" thru_hole circle (at -1.856155 -1.856155) (size 0.8 0.8) (drill 0.5) (layers *.Cu *.Mask) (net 2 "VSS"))
  (pad "1" thru_hole circle (at 2.625 0) (size 0.8 0.8) (drill 0.5) (layers *.Cu *.Mask) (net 2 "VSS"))
  (pad "1" thru_hole circle (at 0 2.625) (size 0.8 0.8) (drill 0.5) (layers *.Cu *.Mask) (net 2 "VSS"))
  (pad "1" thru_hole circle (at 1.856155 -1.856155) (size 0.8 0.8) (drill 0.5) (layers *.Cu *.Mask) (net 2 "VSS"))
  (pad "1" thru_hole circle (at -1.856155 1.856155) (size 0.8 0.8) (drill 0.5) (layers *.Cu *.Mask) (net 2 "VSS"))
  (pad "1" thru_hole circle (at -2.625 0) (size 0.8 0.8) (drill 0.5) (layers *.Cu *.Mask) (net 2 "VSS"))
  (pad "1" thru_hole circle (at 1.856155 1.856155) (size 0.8 0.8) (drill 0.5) (layers *.Cu *.Mask) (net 2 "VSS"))
  (pad "1" thru_hole circle (at 0 0) (size 7 7) (drill 3.5) (layers *.Cu *.Mask) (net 2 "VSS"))
  (pad "1" thru_hole circle (at 0 -2.625) (size 0.8 0.8) (drill 0.5) (layers *.Cu *.Mask) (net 2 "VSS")))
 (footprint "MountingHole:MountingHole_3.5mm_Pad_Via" (layer "F.Cu") (at 147 77.9)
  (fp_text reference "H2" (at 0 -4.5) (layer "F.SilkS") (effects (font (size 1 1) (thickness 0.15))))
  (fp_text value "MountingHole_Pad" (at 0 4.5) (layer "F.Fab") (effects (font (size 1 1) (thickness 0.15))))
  (pad "1" thru_hole circle (at 1.856155 1.856155) (size 0.8 0.8) (drill 0.5) (layers *.Cu *.Mask) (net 2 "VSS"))
  (pad "1" thru_hole circle (at 0 2.625) (size 0.8 0.8) (drill 0.5) (layers *.Cu *.Mask) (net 2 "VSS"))
  (pad "1" thru_hole circle (at -2.625 0) (size 0.8 0.8) (drill 0.5) (layers *.Cu *.Mask) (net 2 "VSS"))
  (pad "1" thru_hole circle (at -1.856155 1.856155) (size 0.8 0.8) (drill 0.5) (layers *.Cu *.Mask) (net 2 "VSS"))
  (pad "1" thru_hole circle (at 2.625 0) (size 0.8 0.8) (drill 0.5) (layers *.Cu *.Mask) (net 2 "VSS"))
  (pad "1" thru_hole circle (at -1.856155 -1.856155) (size 0.8 0.8) (drill 0.5) (layers *.Cu *.Mask) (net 2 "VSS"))
  (pad "1" thru_hole circle (at 0 0) (size 7 7) (drill 3.5) (layers *.Cu *.Mask) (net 2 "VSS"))
  (pad "1" thru_hole circle (at 0 -2.625) (size 0.8 0.8) (drill 0.5) (layers *.Cu *.Mask) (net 2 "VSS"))
  (pad "1" thru_hole circle (at 1.856155 -1.856155) (size 0.8 0.8) (drill 0.5) (layers *.Cu *.Mask) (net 2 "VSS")))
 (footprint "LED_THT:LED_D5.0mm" (layer "F.Cu") (at 145.735 98 180)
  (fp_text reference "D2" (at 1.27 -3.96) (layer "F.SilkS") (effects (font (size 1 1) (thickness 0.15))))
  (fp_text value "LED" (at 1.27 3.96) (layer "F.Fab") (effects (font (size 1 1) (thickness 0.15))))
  (fp_line (start -1.29 -1.545) (end -1.29 1.545) (layer "F.SilkS") (width 0.12))
  (fp_arc (start -1.29 -1.54483) (mid 2.072002 -2.880433) (end 4.26 0.000462) (layer "F.SilkS") (width 0.12))
  (fp_arc (start 4.26 -0.000462) (mid 2.072002 2.880433) (end -1.29 1.54483) (layer "F.SilkS") (width 0.12))
  (fp_circle (center 1.27 0) (end 3.77 0) (layer "F.SilkS") (width 0.12) (fill none))
  (pad "1" thru_hole rect (at 0 0 180) (size 1.8 1.8) (drill 0.9) (layers *.Cu *.Mask) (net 2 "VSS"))
  (pad "2" thru_hole circle (at 2.54 0 180) (size 1.8 1.8) (drill 0.9) (layers *.Cu *.Mask) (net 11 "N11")))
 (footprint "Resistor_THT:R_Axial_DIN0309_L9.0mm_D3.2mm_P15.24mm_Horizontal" (layer "F.Cu") (at 150.37 100.57 90)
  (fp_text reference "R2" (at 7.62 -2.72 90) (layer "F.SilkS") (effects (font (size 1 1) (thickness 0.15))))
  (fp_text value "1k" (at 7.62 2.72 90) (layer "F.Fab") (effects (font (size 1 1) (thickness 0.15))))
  (fp_line (start 3 -1.72) (end 3 1.72) (layer "F.SilkS") (width 0.12))
  (fp_line (start 12.24 1.72) (end 12.24 -1.72) (layer "F.SilkS") (width 0.12))
  (fp_line (start 12.24 -1.72) (end 3 -1.72) (layer "F.SilkS") (width 0.12))
  (fp_line (start 3 1.72) (end 12.24 1.72) (layer "F.SilkS") (width 0.12))
  (fp_line (start 14.2 0) (end 12.24 0) (layer "F.SilkS") (width 0.12))
  (fp_line (start 1.04 0) (end 3 0) (layer "F.SilkS") (width 0.12))
  (pad "1" thru_hole circle (at 0 0 90) (size 1.6 1.6) (drill 0.8) (layers *.Cu *.Mask) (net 5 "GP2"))
  (pad "2" thru_hole oval (at 15.24 0 90) (size 1.6 1.6) (drill 0.8) (layers *.Cu *.Mask) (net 11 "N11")))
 (gr_arc (start 147 72) (mid 151.242641 73.757359) (end 153 78) (layer "Edge.Cuts") (width 0.1))
 (gr_line (start 147 72) (end 117 72) (layer "Edge.Cuts") (width 0.1))
 (gr_line (start 153 78) (end 153 108) (layer "Edge.Cuts") (width 0.1))
 (gr_line (start 111 78) (end 111 108) (layer "Edge.Cuts") (width 0.1))
 (gr_arc (start 111 78) (mid 112.757359 73.757359) (end 117 72) (layer "Edge.Cuts") (width 0.1))
 (gr_arc (start 153 108) (mid 151.242641 112.242641) (end 147 114) (layer "Edge.Cuts") (width 0.1))
 (gr_arc (start 117 114) (mid 112.757359 112.242641) (end 111 108) (layer "Edge.Cuts") (width 0.1))
 (gr_line (start 147 114) (end 117 114) (layer "Edge.Cuts") (width 0.1))
 (segment (start 117 108) (end 120.5 111.5) (width 0.5) (layer "F.Cu") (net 2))
 (segment (start 145.735 98) (end 145.735 106.735) (width 0.5) (layer "F.Cu") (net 2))
 (segment (start 122.52 93.16) (end 121.6 94.08) (width 0.5) (layer "F.Cu") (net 2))
 (segment (start 121.6 94.08) (end 117 89.48) (width 0.5) (layer "F.Cu") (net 2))
 (segment (start 117 77.9) (end 120.5 74.4) (width 0.5) (layer "F.Cu") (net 2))
 (segment (start 145.835 79.065) (end 147 77.9) (width 0.5) (layer "F.Cu") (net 2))
 (segment (start 120.5 111.5) (end 143.5 111.5) (width 0.5) (layer "F.Cu") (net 2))
 (segment (start 143.5 111.5) (end 147 108) (width 0.5) (layer "F.Cu") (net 2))
 (segment (start 147.9 107.1) (end 147 108) (width 0.5) (layer "F.Cu") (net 2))
 (segment (start 134.25 104.25) (end 138 108) (width 0.5) (layer "F.Cu") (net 2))
 (segment (start 129.74 86.26) (end 134.25 81.75) (width 0.5) (layer "F.Cu") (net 2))
 (segment (start 120.5 74.4) (end 143.5 74.4) (width 0.5) (layer "F.Cu") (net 2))
 (segment (start 125.77 93.16) (end 122.52 93.16) (width 0.5) (layer "F.Cu") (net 2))
 (segment (start 143.5 74.4) (end 147 77.9) (width 0.5) (layer "F.Cu") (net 2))
 (segment (start 117 89.48) (end 117 77.9) (width 0.5) (layer "F.Cu") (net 2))
 (segment (start 138 108) (end 147 108) (width 0.5) (layer "F.Cu") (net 2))
 (segment (start 148 78.9) (end 147 77.9) (width 0.5) (layer "F.Cu") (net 2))
 (segment (start 129.74 89.18) (end 129.74 86.26) (width 0.5) (layer "F.Cu") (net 2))
 (segment (start 145.735 106.735) (end 147 108) (width 0.5) (layer "F.Cu") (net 2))
 (segment (start 145.835 88.4) (end 145.835 79.065) (width 0.5) (layer "F.Cu") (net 2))
 (via (at 125.77 93.16) (size 0.8) (drill 0.4) (layers "F.Cu" "B.Cu") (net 2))
 (segment (start 125.77 93.15) (end 125.77 93.16) (width 0.5) (layer "B.Cu") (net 2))
 (segment (start 129.74 89.18) (end 125.77 93.15) (width 0.5) (layer "B.Cu") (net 2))
 (segment (start 138.83 100.62) (end 138.83 97.17) (width 0.5) (layer "F.Cu") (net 9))
 (segment (start 143.295 92.705) (end 143.295 88.4) (width 0.5) (layer "F.Cu") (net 9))
 (segment (start 138.83 97.17) (end 143.295 92.705) (width 0.5) (layer "F.Cu") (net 9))
 (segment (start 138.83 92.79) (end 134.82 96.8) (width 0.5) (layer "F.Cu") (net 6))
 (segment (start 138.83 85.38) (end 138.83 92.79) (width 0.5) (layer "F.Cu") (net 6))
 (segment (start 126.51 84.09) (end 137.54 84.09) (width 0.5) (layer "B.Cu") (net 6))
 (segment (start 137.54 84.09) (end 138.83 85.38) (width 0.5) (layer "B.Cu") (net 6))
 (segment (start 121.6 89) (end 126.51 84.09) (width 0.5) (layer "B.Cu") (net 6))
 (segment (start 134.82 89.18) (end 137 87) (width 0.5) (layer "F.Cu") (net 7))
 (segment (start 137 79.62) (end 139.62 77) (width 0.5) (layer "F.Cu") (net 7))
 (segment (start 132.46 91.54) (end 121.6 91.54) (width 0.5) (layer "F.Cu") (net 7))
 (segment (start 137 87) (end 137 79.62) (width 0.5) (layer "F.Cu") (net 7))
 (segment (start 134.82 89.18) (end 132.46 91.54) (width 0.5) (layer "F.Cu") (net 7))
 (segment (start 127.91 94.97) (end 123.25 94.97) (width 0.5) (layer "F.Cu") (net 4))
 (segment (start 123.25 94.97) (end 121.6 96.62) (width 0.5) (layer "F.Cu") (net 4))
 (segment (start 129.74 96.8) (end 127.91 94.97) (width 0.5) (layer "F.Cu") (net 4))
 (segment (start 124.38 101.94) (end 121.6 99.16) (width 0.5) (layer "F.Cu") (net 8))
 (segment (start 124.38 109) (end 124.38 101.94) (width 0.5) (layer "F.Cu") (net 8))
 (segment (start 124.46 91.92) (end 127.2 89.18) (width 0.5) (layer "B.Cu") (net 8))
 (segment (start 121.6 99.16) (end 124.46 96.3) (width 0.5) (layer "B.Cu") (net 8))
 (segment (start 124.46 96.3) (end 124.46 91.92) (width 0.5) (layer "B.Cu") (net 8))
 (segment (start 138.36 106.08) (end 132.28 100) (width 0.5) (layer "F.Cu") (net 5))
 (segment (start 132.28 100) (end 132.28 96.8) (width 0.5) (layer "F.Cu") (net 5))
 (segment (start 140 106.08) (end 138.36 106.08) (width 0.5) (layer "F.Cu") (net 5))
 (segment (start 127.75 80.37) (end 124.38 77) (width 0.5) (layer "F.Cu") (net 1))
 (segment (start 127.75 81.75) (end 127.75 80.37) (width 0.5) (layer "F.Cu") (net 1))
 (segment (start 127.75 104.25) (end 132.5 109) (width 0.5) (layer "F.Cu") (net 3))
 (segment (start 132.5 109) (end 139.62 109) (width 0.5) (layer "F.Cu") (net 3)))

